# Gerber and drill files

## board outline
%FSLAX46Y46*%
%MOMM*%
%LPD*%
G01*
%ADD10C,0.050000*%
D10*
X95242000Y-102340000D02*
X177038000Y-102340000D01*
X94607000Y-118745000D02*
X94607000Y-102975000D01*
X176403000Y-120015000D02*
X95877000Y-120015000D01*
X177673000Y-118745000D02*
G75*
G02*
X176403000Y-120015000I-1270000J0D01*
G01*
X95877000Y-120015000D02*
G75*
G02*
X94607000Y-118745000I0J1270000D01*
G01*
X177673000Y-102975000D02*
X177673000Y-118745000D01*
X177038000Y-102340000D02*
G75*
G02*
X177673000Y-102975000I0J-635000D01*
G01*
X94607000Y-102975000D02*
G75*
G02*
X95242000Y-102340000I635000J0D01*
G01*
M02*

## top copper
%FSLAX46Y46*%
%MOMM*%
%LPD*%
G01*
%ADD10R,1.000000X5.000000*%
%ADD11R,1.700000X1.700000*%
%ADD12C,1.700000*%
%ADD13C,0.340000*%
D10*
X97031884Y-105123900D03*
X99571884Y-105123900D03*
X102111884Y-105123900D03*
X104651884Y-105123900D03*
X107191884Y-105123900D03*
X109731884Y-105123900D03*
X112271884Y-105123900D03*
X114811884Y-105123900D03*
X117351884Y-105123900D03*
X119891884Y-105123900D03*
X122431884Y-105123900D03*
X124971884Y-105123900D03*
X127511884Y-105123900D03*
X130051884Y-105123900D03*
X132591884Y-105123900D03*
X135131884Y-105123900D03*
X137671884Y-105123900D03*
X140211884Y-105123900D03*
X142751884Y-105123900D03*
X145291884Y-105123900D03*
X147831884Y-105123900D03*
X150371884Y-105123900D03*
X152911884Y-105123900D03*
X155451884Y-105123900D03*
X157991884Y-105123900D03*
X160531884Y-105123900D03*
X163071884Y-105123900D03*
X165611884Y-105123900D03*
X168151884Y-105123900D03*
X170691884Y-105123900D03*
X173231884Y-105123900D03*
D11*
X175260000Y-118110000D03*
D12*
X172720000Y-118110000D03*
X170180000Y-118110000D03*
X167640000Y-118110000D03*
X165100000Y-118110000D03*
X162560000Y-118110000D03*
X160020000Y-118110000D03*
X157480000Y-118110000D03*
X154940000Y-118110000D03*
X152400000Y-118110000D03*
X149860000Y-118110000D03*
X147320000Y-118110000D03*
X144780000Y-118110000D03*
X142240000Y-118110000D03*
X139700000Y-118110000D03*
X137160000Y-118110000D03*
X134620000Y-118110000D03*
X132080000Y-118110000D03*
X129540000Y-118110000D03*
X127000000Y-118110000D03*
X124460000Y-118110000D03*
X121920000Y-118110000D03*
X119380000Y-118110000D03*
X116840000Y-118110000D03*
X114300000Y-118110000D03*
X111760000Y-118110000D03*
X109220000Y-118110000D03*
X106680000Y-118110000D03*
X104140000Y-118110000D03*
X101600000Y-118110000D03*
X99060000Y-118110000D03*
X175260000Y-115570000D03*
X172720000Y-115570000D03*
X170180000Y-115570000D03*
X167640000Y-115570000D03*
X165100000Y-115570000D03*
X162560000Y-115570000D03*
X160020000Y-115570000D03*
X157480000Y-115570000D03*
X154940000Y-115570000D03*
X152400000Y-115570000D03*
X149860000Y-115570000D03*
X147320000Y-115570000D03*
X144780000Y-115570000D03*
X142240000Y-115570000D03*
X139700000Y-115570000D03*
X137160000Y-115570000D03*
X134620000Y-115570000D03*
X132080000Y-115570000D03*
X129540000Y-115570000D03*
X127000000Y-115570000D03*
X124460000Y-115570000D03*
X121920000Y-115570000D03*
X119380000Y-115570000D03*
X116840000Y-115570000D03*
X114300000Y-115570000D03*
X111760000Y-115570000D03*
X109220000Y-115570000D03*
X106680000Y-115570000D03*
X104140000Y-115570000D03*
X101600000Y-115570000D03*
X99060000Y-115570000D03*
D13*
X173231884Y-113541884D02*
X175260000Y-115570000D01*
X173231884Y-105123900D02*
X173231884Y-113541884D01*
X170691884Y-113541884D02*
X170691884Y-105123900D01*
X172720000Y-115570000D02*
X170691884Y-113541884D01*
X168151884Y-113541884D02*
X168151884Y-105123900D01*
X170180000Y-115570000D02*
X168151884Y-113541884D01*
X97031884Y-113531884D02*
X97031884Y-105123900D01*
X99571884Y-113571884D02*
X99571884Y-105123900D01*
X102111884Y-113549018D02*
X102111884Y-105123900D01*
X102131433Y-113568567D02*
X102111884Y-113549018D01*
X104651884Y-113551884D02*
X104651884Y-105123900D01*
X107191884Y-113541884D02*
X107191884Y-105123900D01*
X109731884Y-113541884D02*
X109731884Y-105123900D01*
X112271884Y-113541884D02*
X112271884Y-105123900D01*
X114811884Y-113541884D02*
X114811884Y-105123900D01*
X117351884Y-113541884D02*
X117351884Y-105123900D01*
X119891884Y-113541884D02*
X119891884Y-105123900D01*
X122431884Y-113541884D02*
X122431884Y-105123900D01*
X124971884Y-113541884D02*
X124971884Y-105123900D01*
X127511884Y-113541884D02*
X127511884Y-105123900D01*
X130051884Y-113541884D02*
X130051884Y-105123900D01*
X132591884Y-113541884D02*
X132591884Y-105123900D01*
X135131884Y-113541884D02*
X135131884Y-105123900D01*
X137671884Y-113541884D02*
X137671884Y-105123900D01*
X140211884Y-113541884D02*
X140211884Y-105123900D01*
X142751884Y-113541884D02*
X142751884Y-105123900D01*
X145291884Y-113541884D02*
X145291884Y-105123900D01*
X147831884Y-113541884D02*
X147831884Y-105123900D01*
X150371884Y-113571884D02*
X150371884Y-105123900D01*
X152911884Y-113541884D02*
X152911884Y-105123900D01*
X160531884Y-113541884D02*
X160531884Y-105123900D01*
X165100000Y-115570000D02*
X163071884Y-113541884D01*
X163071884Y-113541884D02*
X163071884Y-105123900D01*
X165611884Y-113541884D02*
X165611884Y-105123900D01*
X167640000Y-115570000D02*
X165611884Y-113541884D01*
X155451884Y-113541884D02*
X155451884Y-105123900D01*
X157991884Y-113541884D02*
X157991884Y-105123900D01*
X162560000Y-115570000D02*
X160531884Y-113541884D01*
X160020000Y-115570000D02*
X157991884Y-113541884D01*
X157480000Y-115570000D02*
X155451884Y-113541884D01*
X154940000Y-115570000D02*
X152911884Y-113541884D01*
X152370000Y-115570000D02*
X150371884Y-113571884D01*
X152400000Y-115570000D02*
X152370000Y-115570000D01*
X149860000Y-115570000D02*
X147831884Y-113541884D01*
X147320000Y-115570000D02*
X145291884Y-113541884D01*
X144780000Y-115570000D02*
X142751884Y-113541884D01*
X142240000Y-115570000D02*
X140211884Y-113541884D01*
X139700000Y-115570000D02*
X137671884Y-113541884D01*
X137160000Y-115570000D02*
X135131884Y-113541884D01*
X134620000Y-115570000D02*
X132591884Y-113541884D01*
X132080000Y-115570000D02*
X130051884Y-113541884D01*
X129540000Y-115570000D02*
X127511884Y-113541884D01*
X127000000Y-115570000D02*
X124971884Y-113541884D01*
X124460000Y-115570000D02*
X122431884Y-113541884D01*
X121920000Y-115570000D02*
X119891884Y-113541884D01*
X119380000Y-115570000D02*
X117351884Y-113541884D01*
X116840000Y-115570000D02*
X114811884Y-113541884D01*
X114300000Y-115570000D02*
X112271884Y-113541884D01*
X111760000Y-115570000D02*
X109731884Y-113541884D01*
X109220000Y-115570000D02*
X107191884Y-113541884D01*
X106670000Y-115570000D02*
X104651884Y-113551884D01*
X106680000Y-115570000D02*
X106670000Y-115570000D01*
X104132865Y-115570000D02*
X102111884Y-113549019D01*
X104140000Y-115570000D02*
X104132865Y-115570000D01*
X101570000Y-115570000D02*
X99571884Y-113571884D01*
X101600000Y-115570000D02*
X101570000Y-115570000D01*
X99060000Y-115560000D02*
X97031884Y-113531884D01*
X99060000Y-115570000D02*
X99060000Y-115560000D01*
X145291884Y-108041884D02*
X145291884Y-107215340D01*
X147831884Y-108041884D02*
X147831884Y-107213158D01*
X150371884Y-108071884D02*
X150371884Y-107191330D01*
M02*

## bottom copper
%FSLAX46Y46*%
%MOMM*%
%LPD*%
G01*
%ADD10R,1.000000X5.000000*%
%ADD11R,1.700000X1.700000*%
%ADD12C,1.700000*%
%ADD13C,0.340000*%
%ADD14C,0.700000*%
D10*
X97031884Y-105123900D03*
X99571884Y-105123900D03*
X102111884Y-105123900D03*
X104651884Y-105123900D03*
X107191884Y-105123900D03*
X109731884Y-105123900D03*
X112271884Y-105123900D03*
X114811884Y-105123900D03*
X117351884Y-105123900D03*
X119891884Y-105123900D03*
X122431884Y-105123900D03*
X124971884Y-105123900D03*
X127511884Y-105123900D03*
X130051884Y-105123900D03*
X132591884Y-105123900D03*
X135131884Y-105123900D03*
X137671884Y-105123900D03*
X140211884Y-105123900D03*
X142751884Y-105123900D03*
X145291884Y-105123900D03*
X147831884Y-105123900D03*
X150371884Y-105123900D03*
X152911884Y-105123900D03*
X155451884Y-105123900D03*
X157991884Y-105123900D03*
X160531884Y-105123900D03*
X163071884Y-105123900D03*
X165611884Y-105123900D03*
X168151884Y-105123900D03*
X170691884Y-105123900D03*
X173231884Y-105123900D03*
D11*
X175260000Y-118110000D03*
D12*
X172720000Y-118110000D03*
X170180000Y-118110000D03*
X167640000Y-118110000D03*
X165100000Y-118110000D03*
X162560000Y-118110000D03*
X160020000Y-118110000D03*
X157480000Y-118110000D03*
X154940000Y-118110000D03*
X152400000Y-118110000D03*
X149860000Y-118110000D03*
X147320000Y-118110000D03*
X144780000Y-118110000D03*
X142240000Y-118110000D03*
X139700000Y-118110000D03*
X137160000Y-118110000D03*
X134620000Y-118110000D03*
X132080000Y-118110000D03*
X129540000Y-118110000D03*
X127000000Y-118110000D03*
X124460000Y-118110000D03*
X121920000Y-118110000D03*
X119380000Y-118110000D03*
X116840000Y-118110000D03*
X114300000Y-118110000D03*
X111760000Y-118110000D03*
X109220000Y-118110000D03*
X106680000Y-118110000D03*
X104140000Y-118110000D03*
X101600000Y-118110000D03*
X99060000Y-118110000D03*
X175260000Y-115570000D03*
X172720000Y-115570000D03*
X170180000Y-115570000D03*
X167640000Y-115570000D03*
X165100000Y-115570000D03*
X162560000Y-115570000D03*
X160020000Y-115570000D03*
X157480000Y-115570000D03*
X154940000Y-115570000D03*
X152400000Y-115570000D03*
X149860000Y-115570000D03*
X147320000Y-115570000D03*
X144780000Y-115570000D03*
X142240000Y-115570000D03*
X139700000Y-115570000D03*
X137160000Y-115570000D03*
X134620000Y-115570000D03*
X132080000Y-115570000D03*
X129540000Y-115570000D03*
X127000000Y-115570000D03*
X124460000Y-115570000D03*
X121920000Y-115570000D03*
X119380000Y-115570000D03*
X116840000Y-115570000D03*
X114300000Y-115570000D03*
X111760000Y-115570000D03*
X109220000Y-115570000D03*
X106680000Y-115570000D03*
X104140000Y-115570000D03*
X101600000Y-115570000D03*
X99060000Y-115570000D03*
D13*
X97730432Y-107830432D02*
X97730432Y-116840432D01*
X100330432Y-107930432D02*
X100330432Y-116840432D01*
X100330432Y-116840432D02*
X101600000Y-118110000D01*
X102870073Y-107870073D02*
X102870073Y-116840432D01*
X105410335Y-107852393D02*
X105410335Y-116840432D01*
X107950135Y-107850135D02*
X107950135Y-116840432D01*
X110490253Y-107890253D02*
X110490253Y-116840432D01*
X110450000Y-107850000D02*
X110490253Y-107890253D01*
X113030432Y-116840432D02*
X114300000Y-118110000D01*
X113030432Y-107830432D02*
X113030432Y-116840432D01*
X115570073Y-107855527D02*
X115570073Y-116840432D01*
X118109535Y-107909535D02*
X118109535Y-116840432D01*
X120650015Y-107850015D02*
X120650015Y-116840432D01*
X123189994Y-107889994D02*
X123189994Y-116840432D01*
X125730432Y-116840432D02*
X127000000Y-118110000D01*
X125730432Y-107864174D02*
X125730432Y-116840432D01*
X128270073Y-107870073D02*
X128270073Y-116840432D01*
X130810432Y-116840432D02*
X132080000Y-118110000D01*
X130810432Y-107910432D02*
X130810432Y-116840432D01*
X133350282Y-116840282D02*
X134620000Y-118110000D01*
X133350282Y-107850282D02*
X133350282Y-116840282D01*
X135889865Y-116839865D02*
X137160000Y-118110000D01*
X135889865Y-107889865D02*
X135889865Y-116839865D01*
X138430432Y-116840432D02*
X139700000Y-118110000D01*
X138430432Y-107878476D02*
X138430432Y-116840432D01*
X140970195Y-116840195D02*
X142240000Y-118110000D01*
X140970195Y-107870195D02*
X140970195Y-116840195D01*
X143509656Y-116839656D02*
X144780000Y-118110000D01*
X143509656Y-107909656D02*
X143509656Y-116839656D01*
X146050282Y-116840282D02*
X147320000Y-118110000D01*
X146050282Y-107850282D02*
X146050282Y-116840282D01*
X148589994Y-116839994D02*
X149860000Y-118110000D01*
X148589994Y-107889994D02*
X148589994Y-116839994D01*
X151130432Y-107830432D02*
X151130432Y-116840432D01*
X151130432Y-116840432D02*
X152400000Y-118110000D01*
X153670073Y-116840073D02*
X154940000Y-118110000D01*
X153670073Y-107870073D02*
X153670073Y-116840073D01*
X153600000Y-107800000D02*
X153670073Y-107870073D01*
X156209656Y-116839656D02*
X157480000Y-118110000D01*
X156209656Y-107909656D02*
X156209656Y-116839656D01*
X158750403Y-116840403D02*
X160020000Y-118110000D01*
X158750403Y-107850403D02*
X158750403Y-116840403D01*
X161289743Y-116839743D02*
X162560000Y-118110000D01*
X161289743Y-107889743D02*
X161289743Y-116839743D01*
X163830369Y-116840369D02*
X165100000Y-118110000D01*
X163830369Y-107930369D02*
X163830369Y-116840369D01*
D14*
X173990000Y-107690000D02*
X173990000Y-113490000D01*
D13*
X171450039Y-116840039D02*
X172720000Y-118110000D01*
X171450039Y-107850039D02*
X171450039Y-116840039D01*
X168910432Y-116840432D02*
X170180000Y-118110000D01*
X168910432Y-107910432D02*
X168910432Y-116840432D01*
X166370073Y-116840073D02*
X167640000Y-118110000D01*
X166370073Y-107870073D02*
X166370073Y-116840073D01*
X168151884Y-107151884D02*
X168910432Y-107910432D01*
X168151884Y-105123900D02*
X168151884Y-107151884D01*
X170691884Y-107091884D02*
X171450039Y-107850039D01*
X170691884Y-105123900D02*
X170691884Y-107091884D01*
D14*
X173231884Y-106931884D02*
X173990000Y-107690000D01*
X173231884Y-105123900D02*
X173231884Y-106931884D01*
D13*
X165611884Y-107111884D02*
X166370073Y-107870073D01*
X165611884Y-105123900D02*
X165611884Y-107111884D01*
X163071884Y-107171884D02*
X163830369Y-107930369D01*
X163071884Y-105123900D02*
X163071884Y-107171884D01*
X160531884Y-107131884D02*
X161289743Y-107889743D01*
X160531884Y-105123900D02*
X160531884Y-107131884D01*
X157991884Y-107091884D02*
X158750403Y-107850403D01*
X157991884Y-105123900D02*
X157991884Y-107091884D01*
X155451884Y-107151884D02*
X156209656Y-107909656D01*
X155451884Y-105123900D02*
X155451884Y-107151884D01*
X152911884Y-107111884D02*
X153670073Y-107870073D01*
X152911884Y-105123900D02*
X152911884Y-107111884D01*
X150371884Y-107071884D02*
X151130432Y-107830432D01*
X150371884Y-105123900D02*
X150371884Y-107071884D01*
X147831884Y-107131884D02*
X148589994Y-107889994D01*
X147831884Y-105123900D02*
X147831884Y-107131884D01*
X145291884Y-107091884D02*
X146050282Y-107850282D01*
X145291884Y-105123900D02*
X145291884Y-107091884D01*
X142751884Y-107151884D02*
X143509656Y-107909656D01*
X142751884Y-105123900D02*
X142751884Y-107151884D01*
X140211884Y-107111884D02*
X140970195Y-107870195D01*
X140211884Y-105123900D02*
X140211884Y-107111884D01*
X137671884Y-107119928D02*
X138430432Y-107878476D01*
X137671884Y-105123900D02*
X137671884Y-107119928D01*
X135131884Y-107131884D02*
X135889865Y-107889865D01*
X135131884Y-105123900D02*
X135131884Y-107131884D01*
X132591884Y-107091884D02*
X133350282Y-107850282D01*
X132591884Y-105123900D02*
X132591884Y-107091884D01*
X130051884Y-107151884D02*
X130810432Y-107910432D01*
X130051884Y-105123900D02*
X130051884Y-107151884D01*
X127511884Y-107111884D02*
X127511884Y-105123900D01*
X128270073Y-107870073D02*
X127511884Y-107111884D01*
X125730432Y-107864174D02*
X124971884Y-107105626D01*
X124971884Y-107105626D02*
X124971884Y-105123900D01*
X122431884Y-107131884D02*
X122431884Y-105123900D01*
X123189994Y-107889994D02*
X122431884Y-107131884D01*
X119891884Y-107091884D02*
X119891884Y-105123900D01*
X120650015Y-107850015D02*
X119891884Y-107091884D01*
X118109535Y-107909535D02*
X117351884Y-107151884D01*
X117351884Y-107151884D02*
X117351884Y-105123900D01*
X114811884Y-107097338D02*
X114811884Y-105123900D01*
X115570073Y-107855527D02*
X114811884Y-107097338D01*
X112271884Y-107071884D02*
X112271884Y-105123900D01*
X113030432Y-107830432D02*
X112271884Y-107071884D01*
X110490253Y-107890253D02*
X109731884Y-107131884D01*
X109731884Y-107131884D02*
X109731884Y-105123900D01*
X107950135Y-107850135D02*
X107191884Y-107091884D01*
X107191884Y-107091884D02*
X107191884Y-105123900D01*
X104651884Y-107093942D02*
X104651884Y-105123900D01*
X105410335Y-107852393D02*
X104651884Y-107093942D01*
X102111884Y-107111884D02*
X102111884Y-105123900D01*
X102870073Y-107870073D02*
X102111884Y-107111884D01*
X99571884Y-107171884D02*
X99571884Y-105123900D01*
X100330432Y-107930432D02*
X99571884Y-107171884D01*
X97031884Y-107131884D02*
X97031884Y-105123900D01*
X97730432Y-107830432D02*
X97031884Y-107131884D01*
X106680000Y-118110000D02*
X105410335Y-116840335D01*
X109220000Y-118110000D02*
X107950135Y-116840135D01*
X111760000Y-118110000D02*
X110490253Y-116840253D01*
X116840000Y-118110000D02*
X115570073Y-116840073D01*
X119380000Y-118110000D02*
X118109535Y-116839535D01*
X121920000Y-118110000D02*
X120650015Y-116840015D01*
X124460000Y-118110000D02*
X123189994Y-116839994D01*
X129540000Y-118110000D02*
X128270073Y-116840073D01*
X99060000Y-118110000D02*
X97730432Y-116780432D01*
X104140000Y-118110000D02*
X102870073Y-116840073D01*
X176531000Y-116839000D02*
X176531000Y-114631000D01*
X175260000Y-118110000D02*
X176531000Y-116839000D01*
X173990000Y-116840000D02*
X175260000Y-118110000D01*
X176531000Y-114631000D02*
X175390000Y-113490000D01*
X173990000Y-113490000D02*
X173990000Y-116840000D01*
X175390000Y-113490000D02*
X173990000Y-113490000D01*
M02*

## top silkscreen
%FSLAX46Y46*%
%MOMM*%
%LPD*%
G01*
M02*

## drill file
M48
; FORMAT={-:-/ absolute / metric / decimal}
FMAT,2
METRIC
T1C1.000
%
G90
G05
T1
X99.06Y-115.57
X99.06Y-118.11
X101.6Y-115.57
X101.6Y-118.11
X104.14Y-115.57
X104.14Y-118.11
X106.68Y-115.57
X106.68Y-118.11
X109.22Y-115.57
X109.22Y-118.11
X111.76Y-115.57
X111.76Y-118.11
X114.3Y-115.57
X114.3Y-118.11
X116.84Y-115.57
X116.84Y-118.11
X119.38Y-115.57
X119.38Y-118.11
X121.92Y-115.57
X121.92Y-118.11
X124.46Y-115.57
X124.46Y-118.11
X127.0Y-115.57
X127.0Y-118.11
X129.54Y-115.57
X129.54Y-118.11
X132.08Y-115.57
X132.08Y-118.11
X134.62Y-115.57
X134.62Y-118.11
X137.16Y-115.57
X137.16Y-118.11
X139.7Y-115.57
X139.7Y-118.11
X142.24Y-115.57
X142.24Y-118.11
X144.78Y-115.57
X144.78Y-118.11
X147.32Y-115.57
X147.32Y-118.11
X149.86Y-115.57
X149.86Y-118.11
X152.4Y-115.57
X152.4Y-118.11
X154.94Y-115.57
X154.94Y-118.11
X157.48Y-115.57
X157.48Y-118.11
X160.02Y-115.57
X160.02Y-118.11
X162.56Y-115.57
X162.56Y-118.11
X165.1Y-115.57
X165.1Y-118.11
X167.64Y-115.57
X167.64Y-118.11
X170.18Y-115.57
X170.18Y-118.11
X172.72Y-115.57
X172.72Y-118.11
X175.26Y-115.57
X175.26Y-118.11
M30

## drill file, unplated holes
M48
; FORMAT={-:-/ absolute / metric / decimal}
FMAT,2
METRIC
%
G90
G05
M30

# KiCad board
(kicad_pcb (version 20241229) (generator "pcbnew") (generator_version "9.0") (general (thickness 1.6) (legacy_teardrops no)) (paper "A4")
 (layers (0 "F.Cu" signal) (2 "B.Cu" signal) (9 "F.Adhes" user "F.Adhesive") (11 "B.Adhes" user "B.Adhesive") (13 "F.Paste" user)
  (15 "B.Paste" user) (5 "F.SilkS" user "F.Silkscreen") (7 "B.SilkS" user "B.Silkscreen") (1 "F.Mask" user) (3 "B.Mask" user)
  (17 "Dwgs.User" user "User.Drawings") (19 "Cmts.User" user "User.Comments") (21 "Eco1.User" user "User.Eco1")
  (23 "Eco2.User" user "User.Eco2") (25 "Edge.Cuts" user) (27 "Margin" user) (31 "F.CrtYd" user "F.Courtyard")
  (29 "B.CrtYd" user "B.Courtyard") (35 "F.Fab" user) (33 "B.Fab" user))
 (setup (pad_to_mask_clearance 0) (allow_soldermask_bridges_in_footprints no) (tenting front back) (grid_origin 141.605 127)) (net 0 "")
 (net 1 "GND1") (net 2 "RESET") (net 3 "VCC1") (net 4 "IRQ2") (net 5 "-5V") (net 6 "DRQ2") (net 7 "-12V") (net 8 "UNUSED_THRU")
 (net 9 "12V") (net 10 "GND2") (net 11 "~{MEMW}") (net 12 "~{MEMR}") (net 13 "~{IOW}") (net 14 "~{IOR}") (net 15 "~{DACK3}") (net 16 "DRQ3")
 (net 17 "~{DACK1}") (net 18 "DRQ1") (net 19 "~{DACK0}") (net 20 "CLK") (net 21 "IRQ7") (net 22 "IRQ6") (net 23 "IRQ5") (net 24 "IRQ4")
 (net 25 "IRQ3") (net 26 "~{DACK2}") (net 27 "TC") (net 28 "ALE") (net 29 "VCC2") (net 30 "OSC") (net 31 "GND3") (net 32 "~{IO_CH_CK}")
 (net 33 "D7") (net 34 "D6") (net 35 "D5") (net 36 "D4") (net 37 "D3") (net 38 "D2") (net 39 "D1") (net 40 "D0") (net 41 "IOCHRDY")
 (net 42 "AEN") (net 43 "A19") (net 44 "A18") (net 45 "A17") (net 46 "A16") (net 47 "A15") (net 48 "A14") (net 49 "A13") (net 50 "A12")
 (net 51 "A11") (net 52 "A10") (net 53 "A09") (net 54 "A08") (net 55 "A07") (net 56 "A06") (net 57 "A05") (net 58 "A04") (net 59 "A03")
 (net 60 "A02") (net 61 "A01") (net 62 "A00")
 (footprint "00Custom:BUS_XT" (layer "F.Cu") (at 173.231884 105.1239)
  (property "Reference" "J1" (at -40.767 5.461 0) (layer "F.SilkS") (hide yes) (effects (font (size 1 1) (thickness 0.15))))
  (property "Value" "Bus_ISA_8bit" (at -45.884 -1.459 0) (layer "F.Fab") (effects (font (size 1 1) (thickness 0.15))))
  (pad "1" smd rect (at 0 0) (size 1 5) (layers "B.Cu" "B.Mask") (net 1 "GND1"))
  (pad "2" smd rect (at -2.54 0) (size 1 5) (layers "B.Cu" "B.Mask") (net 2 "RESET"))
  (pad "3" smd rect (at -5.08 0) (size 1 5) (layers "B.Cu" "B.Mask") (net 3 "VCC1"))
  (pad "4" smd rect (at -7.62 0) (size 1 5) (layers "B.Cu" "B.Mask") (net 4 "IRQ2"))
  (pad "5" smd rect (at -10.16 0) (size 1 5) (layers "B.Cu" "B.Mask") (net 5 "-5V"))
  (pad "6" smd rect (at -12.7 0) (size 1 5) (layers "B.Cu" "B.Mask") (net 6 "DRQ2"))
  (pad "7" smd rect (at -15.24 0) (size 1 5) (layers "B.Cu" "B.Mask") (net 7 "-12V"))
  (pad "8" smd rect (at -17.78 0) (size 1 5) (layers "B.Cu" "B.Mask") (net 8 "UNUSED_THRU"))
  (pad "9" smd rect (at -20.32 0) (size 1 5) (layers "B.Cu" "B.Mask") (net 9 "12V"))
  (pad "10" smd rect (at -22.86 0) (size 1 5) (layers "B.Cu" "B.Mask") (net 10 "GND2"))
  (pad "11" smd rect (at -25.4 0) (size 1 5) (layers "B.Cu" "B.Mask") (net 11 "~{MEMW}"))
  (pad "12" smd rect (at -27.94 0) (size 1 5) (layers "B.Cu" "B.Mask") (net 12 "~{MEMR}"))
  (pad "13" smd rect (at -30.48 0) (size 1 5) (layers "B.Cu" "B.Mask") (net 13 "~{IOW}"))
  (pad "14" smd rect (at -33.02 0) (size 1 5) (layers "B.Cu" "B.Mask") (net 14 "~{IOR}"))
  (pad "15" smd rect (at -35.56 0) (size 1 5) (layers "B.Cu" "B.Mask") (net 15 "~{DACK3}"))
  (pad "16" smd rect (at -38.1 0) (size 1 5) (layers "B.Cu" "B.Mask") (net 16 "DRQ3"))
  (pad "17" smd rect (at -40.64 0) (size 1 5) (layers "B.Cu" "B.Mask") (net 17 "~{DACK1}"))
  (pad "18" smd rect (at -43.18 0) (size 1 5) (layers "B.Cu" "B.Mask") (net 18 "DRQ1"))
  (pad "19" smd rect (at -45.72 0) (size 1 5) (layers "B.Cu" "B.Mask") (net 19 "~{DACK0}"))
  (pad "20" smd rect (at -48.26 0) (size 1 5) (layers "B.Cu" "B.Mask") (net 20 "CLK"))
  (pad "21" smd rect (at -50.8 0) (size 1 5) (layers "B.Cu" "B.Mask") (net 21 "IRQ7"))
  (pad "22" smd rect (at -53.34 0) (size 1 5) (layers "B.Cu" "B.Mask") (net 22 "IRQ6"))
  (pad "23" smd rect (at -55.88 0) (size 1 5) (layers "B.Cu" "B.Mask") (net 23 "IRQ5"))
  (pad "24" smd rect (at -58.42 0) (size 1 5) (layers "B.Cu" "B.Mask") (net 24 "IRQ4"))
  (pad "25" smd rect (at -60.96 0) (size 1 5) (layers "B.Cu" "B.Mask") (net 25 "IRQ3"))
  (pad "26" smd rect (at -63.5 0) (size 1 5) (layers "B.Cu" "B.Mask") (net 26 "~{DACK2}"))
  (pad "27" smd rect (at -66.04 0) (size 1 5) (layers "B.Cu" "B.Mask") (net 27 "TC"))
  (pad "28" smd rect (at -68.58 0) (size 1 5) (layers "B.Cu" "B.Mask") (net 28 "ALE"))
  (pad "29" smd rect (at -71.12 0) (size 1 5) (layers "B.Cu" "B.Mask") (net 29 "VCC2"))
  (pad "30" smd rect (at -73.66 0) (size 1 5) (layers "B.Cu" "B.Mask") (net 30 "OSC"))
  (pad "31" smd rect (at -76.2 0) (size 1 5) (layers "B.Cu" "B.Mask") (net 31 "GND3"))
  (pad "32" smd rect (at 0 0) (size 1 5) (layers "F.Cu" "F.Mask") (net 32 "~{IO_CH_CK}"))
  (pad "33" smd rect (at -2.54 0) (size 1 5) (layers "F.Cu" "F.Mask") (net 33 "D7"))
  (pad "34" smd rect (at -5.08 0) (size 1 5) (layers "F.Cu" "F.Mask") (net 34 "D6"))
  (pad "35" smd rect (at -7.62 0) (size 1 5) (layers "F.Cu" "F.Mask") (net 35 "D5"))
  (pad "36" smd rect (at -10.16 0) (size 1 5) (layers "F.Cu" "F.Mask") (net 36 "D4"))
  (pad "37" smd rect (at -12.7 0) (size 1 5) (layers "F.Cu" "F.Mask") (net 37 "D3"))
  (pad "38" smd rect (at -15.24 0) (size 1 5) (layers "F.Cu" "F.Mask") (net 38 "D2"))
  (pad "39" smd rect (at -17.78 0) (size 1 5) (layers "F.Cu" "F.Mask") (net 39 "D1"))
  (pad "40" smd rect (at -20.32 0) (size 1 5) (layers "F.Cu" "F.Mask") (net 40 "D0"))
  (pad "41" smd rect (at -22.86 0) (size 1 5) (layers "F.Cu" "F.Mask") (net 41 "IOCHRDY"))
  (pad "42" smd rect (at -25.4 0) (size 1 5) (layers "F.Cu" "F.Mask") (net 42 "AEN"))
  (pad "43" smd rect (at -27.94 0) (size 1 5) (layers "F.Cu" "F.Mask") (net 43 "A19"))
  (pad "44" smd rect (at -30.48 0) (size 1 5) (layers "F.Cu" "F.Mask") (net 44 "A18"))
  (pad "45" smd rect (at -33.02 0) (size 1 5) (layers "F.Cu" "F.Mask") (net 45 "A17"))
  (pad "46" smd rect (at -35.56 0) (size 1 5) (layers "F.Cu" "F.Mask") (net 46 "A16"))
  (pad "47" smd rect (at -38.1 0) (size 1 5) (layers "F.Cu" "F.Mask") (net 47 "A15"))
  (pad "48" smd rect (at -40.64 0) (size 1 5) (layers "F.Cu" "F.Mask") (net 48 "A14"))
  (pad "49" smd rect (at -43.18 0) (size 1 5) (layers "F.Cu" "F.Mask") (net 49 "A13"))
  (pad "50" smd rect (at -45.72 0) (size 1 5) (layers "F.Cu" "F.Mask") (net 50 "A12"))
  (pad "51" smd rect (at -48.26 0) (size 1 5) (layers "F.Cu" "F.Mask") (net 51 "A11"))
  (pad "52" smd rect (at -50.8 0) (size 1 5) (layers "F.Cu" "F.Mask") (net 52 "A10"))
  (pad "53" smd rect (at -53.34 0) (size 1 5) (layers "F.Cu" "F.Mask") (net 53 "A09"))
  (pad "54" smd rect (at -55.88 0) (size 1 5) (layers "F.Cu" "F.Mask") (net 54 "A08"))
  (pad "55" smd rect (at -58.42 0) (size 1 5) (layers "F.Cu" "F.Mask") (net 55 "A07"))
  (pad "56" smd rect (at -60.96 0) (size 1 5) (layers "F.Cu" "F.Mask") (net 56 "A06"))
  (pad "57" smd rect (at -63.5 0) (size 1 5) (layers "F.Cu" "F.Mask") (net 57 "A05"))
  (pad "58" smd rect (at -66.04 0) (size 1 5) (layers "F.Cu" "F.Mask") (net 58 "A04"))
  (pad "59" smd rect (at -68.58 0) (size 1 5) (layers "F.Cu" "F.Mask") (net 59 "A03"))
  (pad "60" smd rect (at -71.12 0) (size 1 5) (layers "F.Cu" "F.Mask") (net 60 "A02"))
  (pad "61" smd rect (at -73.66 0) (size 1 5) (layers "F.Cu" "F.Mask") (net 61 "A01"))
  (pad "62" smd rect (at -76.2 0) (size 1 5) (layers "F.Cu" "F.Mask") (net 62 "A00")))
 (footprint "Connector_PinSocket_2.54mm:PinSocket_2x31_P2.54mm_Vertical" (layer "B.Cu") (at 175.26 115.57 90)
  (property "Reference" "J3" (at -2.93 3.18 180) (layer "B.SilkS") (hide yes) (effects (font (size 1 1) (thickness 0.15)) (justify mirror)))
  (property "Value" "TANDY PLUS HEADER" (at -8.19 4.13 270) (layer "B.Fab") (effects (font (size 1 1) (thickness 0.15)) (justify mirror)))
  (pad "1" thru_hole rect (at -2.54 0 90) (size 1.7 1.7) (drill 1) (layers "*.Cu" "*.Mask") (remove_unused_layers no) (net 1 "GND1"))
  (pad "2" thru_hole circle (at -2.54 -2.54 90) (size 1.7 1.7) (drill 1) (layers "*.Cu" "*.Mask") (remove_unused_layers no) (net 2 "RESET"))
  (pad "3" thru_hole circle (at -2.54 -5.08 90) (size 1.7 1.7) (drill 1) (layers "*.Cu" "*.Mask") (remove_unused_layers no) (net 3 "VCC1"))
  (pad "4" thru_hole circle (at -2.54 -7.62 90) (size 1.7 1.7) (drill 1) (layers "*.Cu" "*.Mask") (remove_unused_layers no) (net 4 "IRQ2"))
  (pad "5" thru_hole circle (at -2.54 -10.16 90) (size 1.7 1.7) (drill 1) (layers "*.Cu" "*.Mask") (remove_unused_layers no) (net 5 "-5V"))
  (pad "6" thru_hole circle (at -2.54 -12.7 90) (size 1.7 1.7) (drill 1) (layers "*.Cu" "*.Mask") (remove_unused_layers no) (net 6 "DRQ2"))
  (pad "7" thru_hole circle (at -2.54 -15.24 90) (size 1.7 1.7) (drill 1) (layers "*.Cu" "*.Mask") (remove_unused_layers no) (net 7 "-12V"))
  (pad "8" thru_hole circle (at -2.54 -17.78 90) (size 1.7 1.7) (drill 1) (layers "*.Cu" "*.Mask") (remove_unused_layers no)
   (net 8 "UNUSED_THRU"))
  (pad "9" thru_hole circle (at -2.54 -20.32 90) (size 1.7 1.7) (drill 1) (layers "*.Cu" "*.Mask") (remove_unused_layers no) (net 9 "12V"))
  (pad "10" thru_hole circle (at -2.54 -22.86 90) (size 1.7 1.7) (drill 1) (layers "*.Cu" "*.Mask") (remove_unused_layers no)
   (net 10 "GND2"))
  (pad "11" thru_hole circle (at -2.54 -25.4 90) (size 1.7 1.7) (drill 1) (layers "*.Cu" "*.Mask") (remove_unused_layers no)
   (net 11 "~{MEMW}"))
  (pad "12" thru_hole circle (at -2.54 -27.94 90) (size 1.7 1.7) (drill 1) (layers "*.Cu" "*.Mask") (remove_unused_layers no)
   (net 12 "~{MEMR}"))
  (pad "13" thru_hole circle (at -2.54 -30.48 90) (size 1.7 1.7) (drill 1) (layers "*.Cu" "*.Mask") (remove_unused_layers no)
   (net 13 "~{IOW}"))
  (pad "14" thru_hole circle (at -2.54 -33.02 90) (size 1.7 1.7) (drill 1) (layers "*.Cu" "*.Mask") (remove_unused_layers no)
   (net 14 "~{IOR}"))
  (pad "15" thru_hole circle (at -2.54 -35.56 90) (size 1.7 1.7) (drill 1) (layers "*.Cu" "*.Mask") (remove_unused_layers no)
   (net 15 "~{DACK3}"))
  (pad "16" thru_hole circle (at -2.54 -38.1 90) (size 1.7 1.7) (drill 1) (layers "*.Cu" "*.Mask") (remove_unused_layers no) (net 16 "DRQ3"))
  (pad "17" thru_hole circle (at -2.54 -40.64 90) (size 1.7 1.7) (drill 1) (layers "*.Cu" "*.Mask") (remove_unused_layers no)
   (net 17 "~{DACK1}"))
  (pad "18" thru_hole circle (at -2.54 -43.18 90) (size 1.7 1.7) (drill 1) (layers "*.Cu" "*.Mask") (remove_unused_layers no)
   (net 18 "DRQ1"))
  (pad "19" thru_hole circle (at -2.54 -45.72 90) (size 1.7 1.7) (drill 1) (layers "*.Cu" "*.Mask") (remove_unused_layers no)
   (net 19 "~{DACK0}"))
  (pad "20" thru_hole circle (at -2.54 -48.26 90) (size 1.7 1.7) (drill 1) (layers "*.Cu" "*.Mask") (remove_unused_layers no) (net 20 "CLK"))
  (pad "21" thru_hole circle (at -2.54 -50.8 90) (size 1.7 1.7) (drill 1) (layers "*.Cu" "*.Mask") (remove_unused_layers no) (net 21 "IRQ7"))
  (pad "22" thru_hole circle (at -2.54 -53.34 90) (size 1.7 1.7) (drill 1) (layers "*.Cu" "*.Mask") (remove_unused_layers no)
   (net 22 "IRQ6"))
  (pad "23" thru_hole circle (at -2.54 -55.88 90) (size 1.7 1.7) (drill 1) (layers "*.Cu" "*.Mask") (remove_unused_layers no)
   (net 23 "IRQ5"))
  (pad "24" thru_hole circle (at -2.54 -58.42 90) (size 1.7 1.7) (drill 1) (layers "*.Cu" "*.Mask") (remove_unused_layers no)
   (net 24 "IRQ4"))
  (pad "25" thru_hole circle (at -2.54 -60.96 90) (size 1.7 1.7) (drill 1) (layers "*.Cu" "*.Mask") (remove_unused_layers no)
   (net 25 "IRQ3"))
  (pad "26" thru_hole circle (at -2.54 -63.5 90) (size 1.7 1.7) (drill 1) (layers "*.Cu" "*.Mask") (remove_unused_layers no)
   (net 26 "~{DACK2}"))
  (pad "27" thru_hole circle (at -2.54 -66.04 90) (size 1.7 1.7) (drill 1) (layers "*.Cu" "*.Mask") (remove_unused_layers no) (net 27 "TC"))
  (pad "28" thru_hole circle (at -2.54 -68.58 90) (size 1.7 1.7) (drill 1) (layers "*.Cu" "*.Mask") (remove_unused_layers no) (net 28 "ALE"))
  (pad "29" thru_hole circle (at -2.54 -71.12 90) (size 1.7 1.7) (drill 1) (layers "*.Cu" "*.Mask") (remove_unused_layers no)
   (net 29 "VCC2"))
  (pad "30" thru_hole circle (at -2.54 -73.66 90) (size 1.7 1.7) (drill 1) (layers "*.Cu" "*.Mask") (remove_unused_layers no) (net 30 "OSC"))
  (pad "31" thru_hole circle (at -2.54 -76.2 90) (size 1.7 1.7) (drill 1) (layers "*.Cu" "*.Mask") (remove_unused_layers no) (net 31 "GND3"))
  (pad "32" thru_hole circle (at 0 0 90) (size 1.7 1.7) (drill 1) (layers "*.Cu" "*.Mask") (remove_unused_layers no) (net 32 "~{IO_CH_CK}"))
  (pad "33" thru_hole circle (at 0 -2.54 90) (size 1.7 1.7) (drill 1) (layers "*.Cu" "*.Mask") (remove_unused_layers no) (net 33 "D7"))
  (pad "34" thru_hole circle (at 0 -5.08 90) (size 1.7 1.7) (drill 1) (layers "*.Cu" "*.Mask") (remove_unused_layers no) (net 34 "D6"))
  (pad "35" thru_hole circle (at 0 -7.62 90) (size 1.7 1.7) (drill 1) (layers "*.Cu" "*.Mask") (remove_unused_layers no) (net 35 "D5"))
  (pad "36" thru_hole circle (at 0 -10.16 90) (size 1.7 1.7) (drill 1) (layers "*.Cu" "*.Mask") (remove_unused_layers no) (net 36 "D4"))
  (pad "37" thru_hole circle (at 0 -12.7 90) (size 1.7 1.7) (drill 1) (layers "*.Cu" "*.Mask") (remove_unused_layers no) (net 37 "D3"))
  (pad "38" thru_hole circle (at 0 -15.24 90) (size 1.7 1.7) (drill 1) (layers "*.Cu" "*.Mask") (remove_unused_layers no) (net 38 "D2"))
  (pad "39" thru_hole circle (at 0 -17.78 90) (size 1.7 1.7) (drill 1) (layers "*.Cu" "*.Mask") (remove_unused_layers no) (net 39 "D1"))
  (pad "40" thru_hole circle (at 0 -20.32 90) (size 1.7 1.7) (drill 1) (layers "*.Cu" "*.Mask") (remove_unused_layers no) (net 40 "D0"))
  (pad "41" thru_hole circle (at 0 -22.86 90) (size 1.7 1.7) (drill 1) (layers "*.Cu" "*.Mask") (remove_unused_layers no) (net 41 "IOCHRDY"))
  (pad "42" thru_hole circle (at 0 -25.4 90) (size 1.7 1.7) (drill 1) (layers "*.Cu" "*.Mask") (remove_unused_layers no) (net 42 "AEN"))
  (pad "43" thru_hole circle (at 0 -27.94 90) (size 1.7 1.7) (drill 1) (layers "*.Cu" "*.Mask") (remove_unused_layers no) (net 43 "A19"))
  (pad "44" thru_hole circle (at 0 -30.48 90) (size 1.7 1.7) (drill 1) (layers "*.Cu" "*.Mask") (remove_unused_layers no) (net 44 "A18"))
  (pad "45" thru_hole circle (at 0 -33.02 90) (size 1.7 1.7) (drill 1) (layers "*.Cu" "*.Mask") (remove_unused_layers no) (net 45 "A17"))
  (pad "46" thru_hole circle (at 0 -35.56 90) (size 1.7 1.7) (drill 1) (layers "*.Cu" "*.Mask") (remove_unused_layers no) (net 46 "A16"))
  (pad "47" thru_hole circle (at 0 -38.1 90) (size 1.7 1.7) (drill 1) (layers "*.Cu" "*.Mask") (remove_unused_layers no) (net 47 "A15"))
  (pad "48" thru_hole circle (at 0 -40.64 90) (size 1.7 1.7) (drill 1) (layers "*.Cu" "*.Mask") (remove_unused_layers no) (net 48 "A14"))
  (pad "49" thru_hole circle (at 0 -43.18 90) (size 1.7 1.7) (drill 1) (layers "*.Cu" "*.Mask") (remove_unused_layers no) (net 49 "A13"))
  (pad "50" thru_hole circle (at 0 -45.72 90) (size 1.7 1.7) (drill 1) (layers "*.Cu" "*.Mask") (remove_unused_layers no) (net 50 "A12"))
  (pad "51" thru_hole circle (at 0 -48.26 90) (size 1.7 1.7) (drill 1) (layers "*.Cu" "*.Mask") (remove_unused_layers no) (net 51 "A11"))
  (pad "52" thru_hole circle (at 0 -50.8 90) (size 1.7 1.7) (drill 1) (layers "*.Cu" "*.Mask") (remove_unused_layers no) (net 52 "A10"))
  (pad "53" thru_hole circle (at 0 -53.34 90) (size 1.7 1.7) (drill 1) (layers "*.Cu" "*.Mask") (remove_unused_layers no) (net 53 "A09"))
  (pad "54" thru_hole circle (at 0 -55.88 90) (size 1.7 1.7) (drill 1) (layers "*.Cu" "*.Mask") (remove_unused_layers no) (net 54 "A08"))
  (pad "55" thru_hole circle (at 0 -58.42 90) (size 1.7 1.7) (drill 1) (layers "*.Cu" "*.Mask") (remove_unused_layers no) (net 55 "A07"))
  (pad "56" thru_hole circle (at 0 -60.96 90) (size 1.7 1.7) (drill 1) (layers "*.Cu" "*.Mask") (remove_unused_layers no) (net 56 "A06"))
  (pad "57" thru_hole circle (at 0 -63.5 90) (size 1.7 1.7) (drill 1) (layers "*.Cu" "*.Mask") (remove_unused_layers no) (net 57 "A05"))
  (pad "58" thru_hole circle (at 0 -66.04 90) (size 1.7 1.7) (drill 1) (layers "*.Cu" "*.Mask") (remove_unused_layers no) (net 58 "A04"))
  (pad "59" thru_hole circle (at 0 -68.58 90) (size 1.7 1.7) (drill 1) (layers "*.Cu" "*.Mask") (remove_unused_layers no) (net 59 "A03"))
  (pad "60" thru_hole circle (at 0 -71.12 90) (size 1.7 1.7) (drill 1) (layers "*.Cu" "*.Mask") (remove_unused_layers no) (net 60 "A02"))
  (pad "61" thru_hole circle (at 0 -73.66 90) (size 1.7 1.7) (drill 1) (layers "*.Cu" "*.Mask") (remove_unused_layers no) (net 61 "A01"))
  (pad "62" thru_hole circle (at 0 -76.2 90) (size 1.7 1.7) (drill 1) (layers "*.Cu" "*.Mask") (remove_unused_layers no) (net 62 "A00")))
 (gr_line (start 95.242 102.34) (end 177.038 102.34) (stroke (width 0.05) (type solid)) (layer "Edge.Cuts"))
 (gr_line (start 94.607 118.745) (end 94.607 102.975) (stroke (width 0.05) (type solid)) (layer "Edge.Cuts"))
 (gr_line (start 176.403 120.015) (end 95.877 120.015) (stroke (width 0.05) (type solid)) (layer "Edge.Cuts"))
 (gr_arc (start 177.673 118.745) (mid 177.301026 119.643026) (end 176.403 120.015) (stroke (width 0.05) (type solid)) (layer "Edge.Cuts"))
 (gr_arc (start 95.877 120.015) (mid 94.978974 119.643026) (end 94.607 118.745) (stroke (width 0.05) (type solid)) (layer "Edge.Cuts"))
 (gr_line (start 177.673 102.975) (end 177.673 118.745) (stroke (width 0.05) (type solid)) (layer "Edge.Cuts"))
 (gr_arc (start 177.038 102.34) (mid 177.487013 102.525987) (end 177.673 102.975) (stroke (width 0.05) (type solid)) (layer "Edge.Cuts"))
 (gr_arc (start 94.607 102.975) (mid 94.792987 102.525987) (end 95.242 102.34) (stroke (width 0.05) (type solid)) (layer "Edge.Cuts"))
 (segment (start 99.06 115.57) (end 99.06 115.56) (width 0.34) (layer "F.Cu") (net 62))
 (segment (start 97.031884 113.531884) (end 97.031884 105.1239) (width 0.34) (layer "F.Cu") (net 62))
 (segment (start 99.06 115.56) (end 97.031884 113.531884) (width 0.34) (layer "F.Cu") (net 62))
 (segment (start 99.571884 113.571884) (end 99.571884 105.1239) (width 0.34) (layer "F.Cu") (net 61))
 (segment (start 101.57 115.57) (end 99.571884 113.571884) (width 0.34) (layer "F.Cu") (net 61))
 (segment (start 101.6 115.57) (end 101.57 115.57) (width 0.34) (layer "F.Cu") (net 61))
 (segment (start 102.111884 113.549018) (end 102.111884 105.1239) (width 0.34) (layer "F.Cu") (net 60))
 (segment (start 104.14 115.57) (end 104.132865 115.57) (width 0.34) (layer "F.Cu") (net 60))
 (segment (start 104.132865 115.57) (end 102.111884 113.549019) (width 0.34) (layer "F.Cu") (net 60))
 (segment (start 102.131433 113.568567) (end 102.111884 113.549018) (width 0.34) (layer "F.Cu") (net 60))
 (segment (start 106.68 115.57) (end 106.67 115.57) (width 0.34) (layer "F.Cu") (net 59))
 (segment (start 106.67 115.57) (end 104.651884 113.551884) (width 0.34) (layer "F.Cu") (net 59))
 (segment (start 104.651884 113.551884) (end 104.651884 105.1239) (width 0.34) (layer "F.Cu") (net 59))
 (segment (start 109.22 115.57) (end 107.191884 113.541884) (width 0.34) (layer "F.Cu") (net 58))
 (segment (start 107.191884 113.541884) (end 107.191884 105.1239) (width 0.34) (layer "F.Cu") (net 58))
 (segment (start 109.731884 113.541884) (end 109.731884 105.1239) (width 0.34) (layer "F.Cu") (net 57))
 (segment (start 111.76 115.57) (end 109.731884 113.541884) (width 0.34) (layer "F.Cu") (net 57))
 (segment (start 114.3 115.57) (end 112.271884 113.541884) (width 0.34) (layer "F.Cu") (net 56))
 (segment (start 112.271884 113.541884) (end 112.271884 105.1239) (width 0.34) (layer "F.Cu") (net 56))
 (segment (start 116.84 115.57) (end 114.811884 113.541884) (width 0.34) (layer "F.Cu") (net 55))
 (segment (start 114.811884 113.541884) (end 114.811884 105.1239) (width 0.34) (layer "F.Cu") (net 55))
 (segment (start 119.38 115.57) (end 117.351884 113.541884) (width 0.34) (layer "F.Cu") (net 54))
 (segment (start 117.351884 113.541884) (end 117.351884 105.1239) (width 0.34) (layer "F.Cu") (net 54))
 (segment (start 121.92 115.57) (end 119.891884 113.541884) (width 0.34) (layer "F.Cu") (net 53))
 (segment (start 119.891884 113.541884) (end 119.891884 105.1239) (width 0.34) (layer "F.Cu") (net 53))
 (segment (start 124.46 115.57) (end 122.431884 113.541884) (width 0.34) (layer "F.Cu") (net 52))
 (segment (start 122.431884 113.541884) (end 122.431884 105.1239) (width 0.34) (layer "F.Cu") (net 52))
 (segment (start 127 115.57) (end 124.971884 113.541884) (width 0.34) (layer "F.Cu") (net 51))
 (segment (start 124.971884 113.541884) (end 124.971884 105.1239) (width 0.34) (layer "F.Cu") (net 51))
 (segment (start 127.511884 113.541884) (end 127.511884 105.1239) (width 0.34) (layer "F.Cu") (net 50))
 (segment (start 129.54 115.57) (end 127.511884 113.541884) (width 0.34) (layer "F.Cu") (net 50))
 (segment (start 130.051884 113.541884) (end 130.051884 105.1239) (width 0.34) (layer "F.Cu") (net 49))
 (segment (start 132.08 115.57) (end 130.051884 113.541884) (width 0.34) (layer "F.Cu") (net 49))
 (segment (start 132.591884 113.541884) (end 132.591884 105.1239) (width 0.34) (layer "F.Cu") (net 48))
 (segment (start 134.62 115.57) (end 132.591884 113.541884) (width 0.34) (layer "F.Cu") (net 48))
 (segment (start 137.16 115.57) (end 135.131884 113.541884) (width 0.34) (layer "F.Cu") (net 47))
 (segment (start 135.131884 113.541884) (end 135.131884 105.1239) (width 0.34) (layer "F.Cu") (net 47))
 (segment (start 137.671884 113.541884) (end 137.671884 105.1239) (width 0.34) (layer "F.Cu") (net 46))
 (segment (start 139.7 115.57) (end 137.671884 113.541884) (width 0.34) (layer "F.Cu") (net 46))
 (segment (start 142.24 115.57) (end 140.211884 113.541884) (width 0.34) (layer "F.Cu") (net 45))
 (segment (start 140.211884 113.541884) (end 140.211884 105.1239) (width 0.34) (layer "F.Cu") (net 45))
 (segment (start 142.751884 113.541884) (end 142.751884 105.1239) (width 0.34) (layer "F.Cu") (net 44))
 (segment (start 144.78 115.57) (end 142.751884 113.541884) (width 0.34) (layer "F.Cu") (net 44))
 (segment (start 145.291884 113.541884) (end 145.291884 105.1239) (width 0.34) (layer "F.Cu") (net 43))
 (segment (start 147.32 115.57) (end 145.291884 113.541884) (width 0.34) (layer "F.Cu") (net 43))
 (segment (start 145.291884 108.041884) (end 145.291884 107.21534) (width 0.34) (layer "F.Cu") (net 43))
 (segment (start 147.831884 108.041884) (end 147.831884 107.213158) (width 0.34) (layer "F.Cu") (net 42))
 (segment (start 149.86 115.57) (end 147.831884 113.541884) (width 0.34) (layer "F.Cu") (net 42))
 (segment (start 147.831884 113.541884) (end 147.831884 105.1239) (width 0.34) (layer "F.Cu") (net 42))
 (segment (start 150.371884 113.571884) (end 150.371884 105.1239) (width 0.34) (layer "F.Cu") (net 41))
 (segment (start 152.37 115.57) (end 150.371884 113.571884) (width 0.34) (layer "F.Cu") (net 41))
 (segment (start 150.371884 108.071884) (end 150.371884 107.19133) (width 0.34) (layer "F.Cu") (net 41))
 (segment (start 152.4 115.57) (end 152.37 115.57) (width 0.34) (layer "F.Cu") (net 41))
 (segment (start 154.94 115.57) (end 152.911884 113.541884) (width 0.34) (layer "F.Cu") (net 40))
 (segment (start 152.911884 113.541884) (end 152.911884 105.1239) (width 0.34) (layer "F.Cu") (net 40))
 (segment (start 157.48 115.57) (end 155.451884 113.541884) (width 0.34) (layer "F.Cu") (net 39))
 (segment (start 155.451884 113.541884) (end 155.451884 105.1239) (width 0.34) (layer "F.Cu") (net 39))
 (segment (start 157.991884 113.541884) (end 157.991884 105.1239) (width 0.34) (layer "F.Cu") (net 38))
 (segment (start 160.02 115.57) (end 157.991884 113.541884) (width 0.34) (layer "F.Cu") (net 38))
 (segment (start 162.56 115.57) (end 160.531884 113.541884) (width 0.34) (layer "F.Cu") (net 37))
 (segment (start 160.531884 113.541884) (end 160.531884 105.1239) (width 0.34) (layer "F.Cu") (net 37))
 (segment (start 163.071884 113.541884) (end 163.071884 105.1239) (width 0.34) (layer "F.Cu") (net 36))
 (segment (start 165.1 115.57) (end 163.071884 113.541884) (width 0.34) (layer "F.Cu") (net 36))
 (segment (start 165.611884 113.541884) (end 165.611884 105.1239) (width 0.34) (layer "F.Cu") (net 35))
 (segment (start 167.64 115.57) (end 165.611884 113.541884) (width 0.34) (layer "F.Cu") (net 35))
 (segment (start 170.18 115.57) (end 168.151884 113.541884) (width 0.34) (layer "F.Cu") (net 34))
 (segment (start 168.151884 113.541884) (end 168.151884 105.1239) (width 0.34) (layer "F.Cu") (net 34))
 (segment (start 172.72 115.57) (end 170.691884 113.541884) (width 0.34) (layer "F.Cu") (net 33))
 (segment (start 170.691884 113.541884) (end 170.691884 105.1239) (width 0.34) (layer "F.Cu") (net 33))
 (segment (start 173.231884 105.1239) (end 173.231884 113.541884) (width 0.34) (layer "F.Cu") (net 32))
 (segment (start 173.231884 113.541884) (end 175.26 115.57) (width 0.34) (layer "F.Cu") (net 32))
 (segment (start 100.330432 116.840432) (end 101.6 118.11) (width 0.34) (layer "B.Cu") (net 30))
 (segment (start 99.571884 107.171884) (end 99.571884 105.1239) (width 0.34) (layer "B.Cu") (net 30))
 (segment (start 100.330432 107.930432) (end 99.571884 107.171884) (width 0.34) (layer "B.Cu") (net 30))
 (segment (start 100.330432 107.930432) (end 100.330432 116.840432) (width 0.34) (layer "B.Cu") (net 30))
 (segment (start 104.651884 107.093942) (end 104.651884 105.1239) (width 0.34) (layer "B.Cu") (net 28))
 (segment (start 106.68 118.11) (end 105.410335 116.840335) (width 0.34) (layer "B.Cu") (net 28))
 (segment (start 105.410335 107.852393) (end 105.410335 116.840432) (width 0.34) (layer "B.Cu") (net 28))
 (segment (start 105.410335 107.852393) (end 104.651884 107.093942) (width 0.34) (layer "B.Cu") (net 28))
 (segment (start 107.950135 107.850135) (end 107.950135 116.840432) (width 0.34) (layer "B.Cu") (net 27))
 (segment (start 107.191884 107.091884) (end 107.191884 105.1239) (width 0.34) (layer "B.Cu") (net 27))
 (segment (start 109.22 118.11) (end 107.950135 116.840135) (width 0.34) (layer "B.Cu") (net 27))
 (segment (start 107.950135 107.850135) (end 107.191884 107.091884) (width 0.34) (layer "B.Cu") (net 27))
 (segment (start 109.731884 107.131884) (end 109.731884 105.1239) (width 0.34) (layer "B.Cu") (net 26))
 (segment (start 111.76 118.11) (end 110.490253 116.840253) (width 0.34) (layer "B.Cu") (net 26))
 (segment (start 110.490253 107.890253) (end 109.731884 107.131884) (width 0.34) (layer "B.Cu") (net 26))
 (segment (start 110.45 107.85) (end 110.490253 107.890253) (width 0.34) (layer "B.Cu") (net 26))
 (segment (start 110.490253 107.890253) (end 110.490253 116.840432) (width 0.34) (layer "B.Cu") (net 26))
 (segment (start 113.030432 107.830432) (end 112.271884 107.071884) (width 0.34) (layer "B.Cu") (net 25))
 (segment (start 113.030432 116.840432) (end 114.3 118.11) (width 0.34) (layer "B.Cu") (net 25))
 (segment (start 113.030432 107.830432) (end 113.030432 116.840432) (width 0.34) (layer "B.Cu") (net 25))
 (segment (start 112.271884 107.071884) (end 112.271884 105.1239) (width 0.34) (layer "B.Cu") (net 25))
 (segment (start 115.570073 107.855527) (end 114.811884 107.097338) (width 0.34) (layer "B.Cu") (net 24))
 (segment (start 116.84 118.11) (end 115.570073 116.840073) (width 0.34) (layer "B.Cu") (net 24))
 (segment (start 114.811884 107.097338) (end 114.811884 105.1239) (width 0.34) (layer "B.Cu") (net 24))
 (segment (start 115.570073 107.855527) (end 115.570073 116.840432) (width 0.34) (layer "B.Cu") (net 24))
 (segment (start 119.38 118.11) (end 118.109535 116.839535) (width 0.34) (layer "B.Cu") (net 23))
 (segment (start 118.109535 107.909535) (end 117.351884 107.151884) (width 0.34) (layer "B.Cu") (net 23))
 (segment (start 117.351884 107.151884) (end 117.351884 105.1239) (width 0.34) (layer "B.Cu") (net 23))
 (segment (start 118.109535 107.909535) (end 118.109535 116.840432) (width 0.34) (layer "B.Cu") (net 23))
 (segment (start 119.891884 107.091884) (end 119.891884 105.1239) (width 0.34) (layer "B.Cu") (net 22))
 (segment (start 120.650015 107.850015) (end 119.891884 107.091884) (width 0.34) (layer "B.Cu") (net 22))
 (segment (start 120.650015 107.850015) (end 120.650015 116.840432) (width 0.34) (layer "B.Cu") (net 22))
 (segment (start 121.92 118.11) (end 120.650015 116.840015) (width 0.34) (layer "B.Cu") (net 22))
 (segment (start 122.431884 107.131884) (end 122.431884 105.1239) (width 0.34) (layer "B.Cu") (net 21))
 (segment (start 123.189994 107.889994) (end 123.189994 116.840432) (width 0.34) (layer "B.Cu") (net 21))
 (segment (start 124.46 118.11) (end 123.189994 116.839994) (width 0.34) (layer "B.Cu") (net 21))
 (segment (start 123.189994 107.889994) (end 122.431884 107.131884) (width 0.34) (layer "B.Cu") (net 21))
 (segment (start 125.730432 107.864174) (end 125.730432 116.840432) (width 0.34) (layer "B.Cu") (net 20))
 (segment (start 125.730432 107.864174) (end 124.971884 107.105626) (width 0.34) (layer "B.Cu") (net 20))
 (segment (start 125.730432 116.840432) (end 127 118.11) (width 0.34) (layer "B.Cu") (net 20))
 (segment (start 124.971884 107.105626) (end 124.971884 105.1239) (width 0.34) (layer "B.Cu") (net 20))
 (segment (start 128.270073 107.870073) (end 128.270073 116.840432) (width 0.34) (layer "B.Cu") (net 19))
 (segment (start 129.54 118.11) (end 128.270073 116.840073) (width 0.34) (layer "B.Cu") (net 19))
 (segment (start 127.511884 107.111884) (end 127.511884 105.1239) (width 0.34) (layer "B.Cu") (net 19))
 (segment (start 128.270073 107.870073) (end 127.511884 107.111884) (width 0.34) (layer "B.Cu") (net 19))
 (segment (start 130.051884 107.151884) (end 130.810432 107.910432) (width 0.34) (layer "B.Cu") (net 18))
 (segment (start 130.051884 105.1239) (end 130.051884 107.151884) (width 0.34) (layer "B.Cu") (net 18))
 (segment (start 130.810432 116.840432) (end 132.08 118.11) (width 0.34) (layer "B.Cu") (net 18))
 (segment (start 130.810432 107.910432) (end 130.810432 116.840432) (width 0.34) (layer "B.Cu") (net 18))
 (segment (start 133.350282 107.850282) (end 133.350282 116.840282) (width 0.34) (layer "B.Cu") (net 17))
 (segment (start 132.591884 107.091884) (end 133.350282 107.850282) (width 0.34) (layer "B.Cu") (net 17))
 (segment (start 133.350282 116.840282) (end 134.62 118.11) (width 0.34) (layer "B.Cu") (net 17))
 (segment (start 132.591884 105.1239) (end 132.591884 107.091884) (width 0.34) (layer "B.Cu") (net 17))
 (segment (start 135.131884 105.1239) (end 135.131884 107.131884) (width 0.34) (layer "B.Cu") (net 16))
 (segment (start 135.131884 107.131884) (end 135.889865 107.889865) (width 0.34) (layer "B.Cu") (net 16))
 (segment (start 135.889865 107.889865) (end 135.889865 116.839865) (width 0.34) (layer "B.Cu") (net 16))
 (segment (start 135.889865 116.839865) (end 137.16 118.11) (width 0.34) (layer "B.Cu") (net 16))
 (segment (start 137.671884 107.119928) (end 138.430432 107.878476) (width 0.34) (layer "B.Cu") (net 15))
 (segment (start 138.430432 107.878476) (end 138.430432 116.840432) (width 0.34) (layer "B.Cu") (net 15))
 (segment (start 137.671884 105.1239) (end 137.671884 107.119928) (width 0.34) (layer "B.Cu") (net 15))
 (segment (start 138.430432 116.840432) (end 139.7 118.11) (width 0.34) (layer "B.Cu") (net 15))
 (segment (start 140.211884 107.111884) (end 140.970195 107.870195) (width 0.34) (layer "B.Cu") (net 14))
 (segment (start 140.970195 107.870195) (end 140.970195 116.840195) (width 0.34) (layer "B.Cu") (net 14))
 (segment (start 140.970195 116.840195) (end 142.24 118.11) (width 0.34) (layer "B.Cu") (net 14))
 (segment (start 140.211884 105.1239) (end 140.211884 107.111884) (width 0.34) (layer "B.Cu") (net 14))
 (segment (start 143.509656 116.839656) (end 144.78 118.11) (width 0.34) (layer "B.Cu") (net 13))
 (segment (start 142.751884 107.151884) (end 143.509656 107.909656) (width 0.34) (layer "B.Cu") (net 13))
 (segment (start 143.509656 107.909656) (end 143.509656 116.839656) (width 0.34) (layer "B.Cu") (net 13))
 (segment (start 142.751884 105.1239) (end 142.751884 107.151884) (width 0.34) (layer "B.Cu") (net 13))
 (segment (start 145.291884 107.091884) (end 146.050282 107.850282) (width 0.34) (layer "B.Cu") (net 12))
 (segment (start 146.050282 107.850282) (end 146.050282 116.840282) (width 0.34) (layer "B.Cu") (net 12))
 (segment (start 146.050282 116.840282) (end 147.32 118.11) (width 0.34) (layer "B.Cu") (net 12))
 (segment (start 145.291884 105.1239) (end 145.291884 107.091884) (width 0.34) (layer "B.Cu") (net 12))
 (segment (start 147.831884 107.131884) (end 148.589994 107.889994) (width 0.34) (layer "B.Cu") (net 11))
 (segment (start 148.589994 116.839994) (end 149.86 118.11) (width 0.34) (layer "B.Cu") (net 11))
 (segment (start 147.831884 105.1239) (end 147.831884 107.131884) (width 0.34) (layer "B.Cu") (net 11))
 (segment (start 148.589994 107.889994) (end 148.589994 116.839994) (width 0.34) (layer "B.Cu") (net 11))
 (segment (start 158.750403 116.840403) (end 160.02 118.11) (width 0.34) (layer "B.Cu") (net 7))
 (segment (start 157.991884 105.1239) (end 157.991884 107.091884) (width 0.34) (layer "B.Cu") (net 7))
 (segment (start 157.991884 107.091884) (end 158.750403 107.850403) (width 0.34) (layer "B.Cu") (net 7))
 (segment (start 158.750403 107.850403) (end 158.750403 116.840403) (width 0.34) (layer "B.Cu") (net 7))
 (segment (start 160.531884 105.1239) (end 160.531884 107.131884) (width 0.34) (layer "B.Cu") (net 6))
 (segment (start 161.289743 116.839743) (end 162.56 118.11) (width 0.34) (layer "B.Cu") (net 6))
 (segment (start 161.289743 107.889743) (end 161.289743 116.839743) (width 0.34) (layer "B.Cu") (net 6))
 (segment (start 160.531884 107.131884) (end 161.289743 107.889743) (width 0.34) (layer "B.Cu") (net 6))
 (segment (start 163.071884 107.171884) (end 163.830369 107.930369) (width 0.34) (layer "B.Cu") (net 5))
 (segment (start 163.830369 116.840369) (end 165.1 118.11) (width 0.34) (layer "B.Cu") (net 5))
 (segment (start 163.830369 107.930369) (end 163.830369 116.840369) (width 0.34) (layer "B.Cu") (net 5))
 (segment (start 163.071884 105.1239) (end 163.071884 107.171884) (width 0.34) (layer "B.Cu") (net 5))
 (segment (start 166.370073 116.840073) (end 167.64 118.11) (width 0.34) (layer "B.Cu") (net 4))
 (segment (start 165.611884 107.111884) (end 166.370073 107.870073) (width 0.34) (layer "B.Cu") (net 4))
 (segment (start 165.611884 105.1239) (end 165.611884 107.111884) (width 0.34) (layer "B.Cu") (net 4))
 (segment (start 166.370073 107.870073) (end 166.370073 116.840073) (width 0.34) (layer "B.Cu") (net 4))
 (segment (start 171.450039 107.850039) (end 171.450039 116.840039) (width 0.34) (layer "B.Cu") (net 2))
 (segment (start 171.450039 116.840039) (end 172.72 118.11) (width 0.34) (layer "B.Cu") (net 2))
 (segment (start 170.691884 105.1239) (end 170.691884 107.091884) (width 0.34) (layer "B.Cu") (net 2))
 (segment (start 170.691884 107.091884) (end 171.450039 107.850039) (width 0.34) (layer "B.Cu") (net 2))
 (segment (start 97.730432 107.830432) (end 97.730432 116.840432) (width 0.34) (layer "B.Cu") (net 31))
 (segment (start 99.06 118.11) (end 97.730432 116.780432) (width 0.34) (layer "B.Cu") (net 31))
 (segment (start 97.730432 107.830432) (end 97.031884 107.131884) (width 0.34) (layer "B.Cu") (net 31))
 (segment (start 97.031884 107.131884) (end 97.031884 105.1239) (width 0.34) (layer "B.Cu") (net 31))
 (segment (start 102.870073 107.870073) (end 102.111884 107.111884) (width 0.34) (layer "B.Cu") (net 29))
 (segment (start 104.14 118.11) (end 102.870073 116.840073) (width 0.34) (layer "B.Cu") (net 29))
 (segment (start 102.111884 107.111884) (end 102.111884 105.1239) (width 0.34) (layer "B.Cu") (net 29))
 (segment (start 102.870073 107.870073) (end 102.870073 116.840432) (width 0.34) (layer "B.Cu") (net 29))
 (segment (start 150.371884 107.071884) (end 151.130432 107.830432) (width 0.34) (layer "B.Cu") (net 10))
 (segment (start 150.371884 105.1239) (end 150.371884 107.071884) (width 0.34) (layer "B.Cu") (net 10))
 (segment (start 151.130432 107.830432) (end 151.130432 116.840432) (width 0.34) (layer "B.Cu") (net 10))
 (segment (start 151.130432 116.840432) (end 152.4 118.11) (width 0.34) (layer "B.Cu") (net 10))
 (segment (start 153.670073 107.870073) (end 153.670073 116.840073) (width 0.34) (layer "B.Cu") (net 9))
 (segment (start 153.6 107.8) (end 153.670073 107.870073) (width 0.34) (layer "B.Cu") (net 9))
 (segment (start 152.911884 107.111884) (end 153.670073 107.870073) (width 0.34) (layer "B.Cu") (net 9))
 (segment (start 153.670073 116.840073) (end 154.94 118.11) (width 0.34) (layer "B.Cu") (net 9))
 (segment (start 152.911884 105.1239) (end 152.911884 107.111884) (width 0.34) (layer "B.Cu") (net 9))
 (segment (start 155.451884 107.151884) (end 156.209656 107.909656) (width 0.34) (layer "B.Cu") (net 8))
 (segment (start 155.451884 105.1239) (end 155.451884 107.151884) (width 0.34) (layer "B.Cu") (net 8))
 (segment (start 156.209656 116.839656) (end 157.48 118.11) (width 0.34) (layer "B.Cu") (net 8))
 (segment (start 156.209656 107.909656) (end 156.209656 116.839656) (width 0.34) (layer "B.Cu") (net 8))
 (segment (start 168.910432 116.840432) (end 170.18 118.11) (width 0.34) (layer "B.Cu") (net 3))
 (segment (start 168.151884 107.151884) (end 168.910432 107.910432) (width 0.34) (layer "B.Cu") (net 3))
 (segment (start 168.910432 107.910432) (end 168.910432 116.840432) (width 0.34) (layer "B.Cu") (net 3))
 (segment (start 168.151884 105.1239) (end 168.151884 107.151884) (width 0.34) (layer "B.Cu") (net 3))
 (segment (start 173.99 107.69) (end 173.99 113.49) (width 0.7) (layer "B.Cu") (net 1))
 (segment (start 176.531 116.839) (end 176.531 114.631) (width 0.34) (layer "B.Cu") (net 1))
 (segment (start 175.26 118.11) (end 176.531 116.839) (width 0.34) (layer "B.Cu") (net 1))
 (segment (start 173.99 116.84) (end 175.26 118.11) (width 0.34) (layer "B.Cu") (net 1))
 (segment (start 173.231884 106.931884) (end 173.99 107.69) (width 0.7) (layer "B.Cu") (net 1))
 (segment (start 176.531 114.631) (end 175.39 113.49) (width 0.34) (layer "B.Cu") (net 1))
 (segment (start 173.99 113.49) (end 173.99 116.84) (width 0.34) (layer "B.Cu") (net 1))
 (segment (start 173.231884 105.1239) (end 173.231884 106.931884) (width 0.7) (layer "B.Cu") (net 1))
 (segment (start 175.39 113.49) (end 173.99 113.49) (width 0.34) (layer "B.Cu") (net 1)))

